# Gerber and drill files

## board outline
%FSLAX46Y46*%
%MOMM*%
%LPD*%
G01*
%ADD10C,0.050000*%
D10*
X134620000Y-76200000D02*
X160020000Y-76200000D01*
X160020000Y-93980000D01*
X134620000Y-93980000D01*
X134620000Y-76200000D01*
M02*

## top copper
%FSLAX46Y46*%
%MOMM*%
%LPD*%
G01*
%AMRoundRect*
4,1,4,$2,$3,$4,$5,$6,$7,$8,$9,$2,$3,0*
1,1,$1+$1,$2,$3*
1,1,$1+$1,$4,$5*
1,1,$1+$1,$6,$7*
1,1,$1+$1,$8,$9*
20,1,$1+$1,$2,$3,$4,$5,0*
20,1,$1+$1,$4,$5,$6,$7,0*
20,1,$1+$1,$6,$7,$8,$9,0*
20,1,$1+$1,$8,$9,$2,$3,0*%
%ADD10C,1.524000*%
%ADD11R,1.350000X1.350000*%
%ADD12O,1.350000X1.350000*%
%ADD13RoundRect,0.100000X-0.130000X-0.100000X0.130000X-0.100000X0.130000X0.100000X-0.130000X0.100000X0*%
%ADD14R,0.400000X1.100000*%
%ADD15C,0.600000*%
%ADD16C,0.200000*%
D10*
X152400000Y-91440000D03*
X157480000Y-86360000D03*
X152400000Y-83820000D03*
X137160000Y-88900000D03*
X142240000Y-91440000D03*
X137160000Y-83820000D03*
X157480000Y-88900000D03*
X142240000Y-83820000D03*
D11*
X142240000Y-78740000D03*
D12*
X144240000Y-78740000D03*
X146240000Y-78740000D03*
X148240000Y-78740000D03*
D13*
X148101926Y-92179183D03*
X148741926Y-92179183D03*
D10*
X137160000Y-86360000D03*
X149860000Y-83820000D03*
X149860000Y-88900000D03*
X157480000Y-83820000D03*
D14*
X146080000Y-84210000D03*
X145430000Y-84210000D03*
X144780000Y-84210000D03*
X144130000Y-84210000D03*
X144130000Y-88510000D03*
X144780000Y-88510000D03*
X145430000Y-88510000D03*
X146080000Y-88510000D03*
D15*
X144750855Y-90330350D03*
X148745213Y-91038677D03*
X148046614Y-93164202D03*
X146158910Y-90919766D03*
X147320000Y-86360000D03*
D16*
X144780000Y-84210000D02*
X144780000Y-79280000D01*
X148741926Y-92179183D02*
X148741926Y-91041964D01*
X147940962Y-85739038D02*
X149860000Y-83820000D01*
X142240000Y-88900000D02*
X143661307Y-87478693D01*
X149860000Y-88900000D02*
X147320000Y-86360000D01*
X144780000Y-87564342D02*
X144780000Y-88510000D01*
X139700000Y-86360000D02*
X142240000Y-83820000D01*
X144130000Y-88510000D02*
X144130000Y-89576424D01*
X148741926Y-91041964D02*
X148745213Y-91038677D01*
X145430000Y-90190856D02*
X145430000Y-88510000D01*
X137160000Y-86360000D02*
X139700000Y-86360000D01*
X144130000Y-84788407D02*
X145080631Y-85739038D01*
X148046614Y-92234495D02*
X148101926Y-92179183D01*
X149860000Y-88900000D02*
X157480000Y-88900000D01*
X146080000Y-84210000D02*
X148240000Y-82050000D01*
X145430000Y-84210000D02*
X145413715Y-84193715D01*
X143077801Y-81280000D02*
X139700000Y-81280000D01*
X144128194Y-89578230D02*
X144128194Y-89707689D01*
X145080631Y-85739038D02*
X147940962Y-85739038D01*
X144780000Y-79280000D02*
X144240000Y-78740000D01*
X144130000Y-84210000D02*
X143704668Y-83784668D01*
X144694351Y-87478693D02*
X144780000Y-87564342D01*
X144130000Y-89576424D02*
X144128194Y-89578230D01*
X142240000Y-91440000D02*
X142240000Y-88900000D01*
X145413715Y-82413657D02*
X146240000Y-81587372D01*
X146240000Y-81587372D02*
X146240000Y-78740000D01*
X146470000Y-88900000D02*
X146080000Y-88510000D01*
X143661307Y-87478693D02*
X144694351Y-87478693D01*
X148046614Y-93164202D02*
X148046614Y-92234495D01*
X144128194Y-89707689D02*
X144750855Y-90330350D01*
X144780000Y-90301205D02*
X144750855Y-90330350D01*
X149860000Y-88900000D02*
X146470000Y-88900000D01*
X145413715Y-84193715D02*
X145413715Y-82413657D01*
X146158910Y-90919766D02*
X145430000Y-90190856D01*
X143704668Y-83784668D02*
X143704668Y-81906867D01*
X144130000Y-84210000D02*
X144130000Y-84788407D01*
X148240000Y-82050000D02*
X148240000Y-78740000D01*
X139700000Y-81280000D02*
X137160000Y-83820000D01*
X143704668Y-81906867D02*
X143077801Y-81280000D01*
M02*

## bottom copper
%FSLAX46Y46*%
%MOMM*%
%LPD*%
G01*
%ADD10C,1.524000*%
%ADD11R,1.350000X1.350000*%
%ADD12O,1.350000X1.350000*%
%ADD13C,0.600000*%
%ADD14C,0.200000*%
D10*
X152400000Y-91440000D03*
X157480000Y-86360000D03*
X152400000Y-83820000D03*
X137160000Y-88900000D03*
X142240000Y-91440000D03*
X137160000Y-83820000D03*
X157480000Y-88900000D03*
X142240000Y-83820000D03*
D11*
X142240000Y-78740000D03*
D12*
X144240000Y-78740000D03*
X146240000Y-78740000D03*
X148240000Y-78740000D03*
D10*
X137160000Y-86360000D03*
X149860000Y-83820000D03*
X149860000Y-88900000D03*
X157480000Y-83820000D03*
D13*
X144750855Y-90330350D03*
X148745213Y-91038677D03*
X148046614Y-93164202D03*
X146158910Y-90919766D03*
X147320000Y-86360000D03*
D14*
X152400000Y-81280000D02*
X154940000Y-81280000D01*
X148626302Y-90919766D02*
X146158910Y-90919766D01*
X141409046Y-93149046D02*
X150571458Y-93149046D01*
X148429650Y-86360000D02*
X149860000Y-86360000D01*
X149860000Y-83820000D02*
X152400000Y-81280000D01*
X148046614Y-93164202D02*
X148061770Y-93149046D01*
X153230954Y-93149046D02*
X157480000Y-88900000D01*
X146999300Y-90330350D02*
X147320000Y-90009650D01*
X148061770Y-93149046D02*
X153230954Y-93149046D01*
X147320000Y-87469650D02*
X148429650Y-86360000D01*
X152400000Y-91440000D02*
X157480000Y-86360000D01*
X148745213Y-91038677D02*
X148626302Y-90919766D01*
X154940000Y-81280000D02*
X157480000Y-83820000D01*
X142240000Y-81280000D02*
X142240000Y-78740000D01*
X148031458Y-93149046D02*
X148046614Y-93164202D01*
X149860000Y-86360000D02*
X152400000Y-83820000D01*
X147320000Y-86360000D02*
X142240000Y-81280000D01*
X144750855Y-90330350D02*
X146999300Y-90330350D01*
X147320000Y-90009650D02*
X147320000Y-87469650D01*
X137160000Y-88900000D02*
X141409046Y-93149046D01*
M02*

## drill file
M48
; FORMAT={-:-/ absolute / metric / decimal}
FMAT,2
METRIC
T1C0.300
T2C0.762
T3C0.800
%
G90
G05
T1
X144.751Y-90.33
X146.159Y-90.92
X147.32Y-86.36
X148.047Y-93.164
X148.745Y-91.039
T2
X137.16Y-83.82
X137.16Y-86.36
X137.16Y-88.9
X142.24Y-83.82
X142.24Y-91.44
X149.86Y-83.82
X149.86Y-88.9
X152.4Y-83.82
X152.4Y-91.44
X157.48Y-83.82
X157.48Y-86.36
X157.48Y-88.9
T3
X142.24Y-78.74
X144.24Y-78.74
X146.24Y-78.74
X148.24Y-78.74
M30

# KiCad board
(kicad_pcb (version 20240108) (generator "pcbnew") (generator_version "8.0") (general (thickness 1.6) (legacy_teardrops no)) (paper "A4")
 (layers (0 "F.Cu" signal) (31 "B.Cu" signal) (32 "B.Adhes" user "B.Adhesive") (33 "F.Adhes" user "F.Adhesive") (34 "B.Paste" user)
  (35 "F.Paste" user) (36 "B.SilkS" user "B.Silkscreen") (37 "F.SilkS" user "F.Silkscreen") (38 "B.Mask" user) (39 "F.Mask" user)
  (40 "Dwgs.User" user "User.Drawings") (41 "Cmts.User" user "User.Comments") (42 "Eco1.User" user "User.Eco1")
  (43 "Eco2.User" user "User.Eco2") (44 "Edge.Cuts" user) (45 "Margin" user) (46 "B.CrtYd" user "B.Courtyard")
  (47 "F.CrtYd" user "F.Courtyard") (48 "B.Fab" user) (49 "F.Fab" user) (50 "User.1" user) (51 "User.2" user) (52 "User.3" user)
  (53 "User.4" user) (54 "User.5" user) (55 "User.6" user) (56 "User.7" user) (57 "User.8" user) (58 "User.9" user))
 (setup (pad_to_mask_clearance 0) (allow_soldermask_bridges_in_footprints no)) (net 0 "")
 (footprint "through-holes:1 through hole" (layer "F.Cu") (at 152.4 91.44)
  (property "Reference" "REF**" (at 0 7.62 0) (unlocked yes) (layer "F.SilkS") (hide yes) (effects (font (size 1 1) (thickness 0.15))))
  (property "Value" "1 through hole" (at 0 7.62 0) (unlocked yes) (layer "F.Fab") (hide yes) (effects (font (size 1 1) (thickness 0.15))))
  (pad "1" thru_hole circle (at 0 0) (size 1.524 1.524) (drill 0.762) (layers "*.Cu" "*.Mask") (remove_unused_layers no)))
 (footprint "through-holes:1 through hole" (layer "F.Cu") (at 157.48 86.36)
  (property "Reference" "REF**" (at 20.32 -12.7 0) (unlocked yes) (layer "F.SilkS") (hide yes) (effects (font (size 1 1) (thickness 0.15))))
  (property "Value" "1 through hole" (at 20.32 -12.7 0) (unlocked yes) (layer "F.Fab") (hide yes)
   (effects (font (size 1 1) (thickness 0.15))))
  (pad "1" thru_hole circle (at 0 0) (size 1.524 1.524) (drill 0.762) (layers "*.Cu" "*.Mask") (remove_unused_layers no)))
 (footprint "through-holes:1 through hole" (layer "F.Cu") (at 152.4 83.82)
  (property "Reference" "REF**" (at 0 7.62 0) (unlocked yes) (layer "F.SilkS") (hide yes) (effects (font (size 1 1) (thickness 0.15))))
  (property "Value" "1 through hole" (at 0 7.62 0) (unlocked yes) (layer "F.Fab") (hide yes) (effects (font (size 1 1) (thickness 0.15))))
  (pad "1" thru_hole circle (at 0 0) (size 1.524 1.524) (drill 0.762) (layers "*.Cu" "*.Mask") (remove_unused_layers no)))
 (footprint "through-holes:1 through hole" (layer "F.Cu") (at 137.16 88.9)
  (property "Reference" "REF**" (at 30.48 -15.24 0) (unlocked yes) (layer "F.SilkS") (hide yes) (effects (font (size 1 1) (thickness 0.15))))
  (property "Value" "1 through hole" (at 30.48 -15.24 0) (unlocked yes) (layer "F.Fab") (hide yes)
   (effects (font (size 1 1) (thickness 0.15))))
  (pad "1" thru_hole circle (at 0 0) (size 1.524 1.524) (drill 0.762) (layers "*.Cu" "*.Mask") (remove_unused_layers no)))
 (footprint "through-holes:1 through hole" (layer "F.Cu") (at 142.24 91.44)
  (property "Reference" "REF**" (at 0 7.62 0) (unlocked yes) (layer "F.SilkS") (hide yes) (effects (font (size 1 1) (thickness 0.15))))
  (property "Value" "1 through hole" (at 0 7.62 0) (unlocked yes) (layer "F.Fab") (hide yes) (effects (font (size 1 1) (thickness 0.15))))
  (pad "1" thru_hole circle (at 0 0) (size 1.524 1.524) (drill 0.762) (layers "*.Cu" "*.Mask") (remove_unused_layers no)))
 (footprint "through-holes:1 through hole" (layer "F.Cu") (at 137.16 83.82)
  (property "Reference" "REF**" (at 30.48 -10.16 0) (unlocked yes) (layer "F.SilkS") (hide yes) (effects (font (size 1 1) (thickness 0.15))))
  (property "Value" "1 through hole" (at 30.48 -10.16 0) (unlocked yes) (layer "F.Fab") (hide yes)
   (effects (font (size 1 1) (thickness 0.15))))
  (pad "1" thru_hole circle (at 0 0) (size 1.524 1.524) (drill 0.762) (layers "*.Cu" "*.Mask") (remove_unused_layers no)))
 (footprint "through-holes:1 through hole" (layer "F.Cu") (at 157.48 88.9)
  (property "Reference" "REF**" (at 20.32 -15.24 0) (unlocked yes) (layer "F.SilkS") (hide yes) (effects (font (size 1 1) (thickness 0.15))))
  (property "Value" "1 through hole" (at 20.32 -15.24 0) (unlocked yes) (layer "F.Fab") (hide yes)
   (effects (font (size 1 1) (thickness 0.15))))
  (pad "1" thru_hole circle (at 0 0) (size 1.524 1.524) (drill 0.762) (layers "*.Cu" "*.Mask") (remove_unused_layers no)))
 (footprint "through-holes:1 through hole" (layer "F.Cu") (at 142.24 83.82)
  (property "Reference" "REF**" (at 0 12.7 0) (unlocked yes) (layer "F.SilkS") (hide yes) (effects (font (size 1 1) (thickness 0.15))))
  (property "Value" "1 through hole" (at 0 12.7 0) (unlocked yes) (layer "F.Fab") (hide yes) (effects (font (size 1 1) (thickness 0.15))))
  (pad "1" thru_hole circle (at 0 0) (size 1.524 1.524) (drill 0.762) (layers "*.Cu" "*.Mask") (remove_unused_layers no)))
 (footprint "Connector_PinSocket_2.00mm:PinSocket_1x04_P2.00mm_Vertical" (layer "F.Cu") (at 142.24 78.74 90)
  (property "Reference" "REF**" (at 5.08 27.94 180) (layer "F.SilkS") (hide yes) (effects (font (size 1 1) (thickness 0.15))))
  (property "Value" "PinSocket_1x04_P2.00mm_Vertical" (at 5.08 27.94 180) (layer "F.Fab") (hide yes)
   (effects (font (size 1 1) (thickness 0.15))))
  (pad "1" thru_hole rect (at 0 0 90) (size 1.35 1.35) (drill 0.8) (layers "*.Cu" "*.Mask") (remove_unused_layers no))
  (pad "2" thru_hole oval (at 0 2 90) (size 1.35 1.35) (drill 0.8) (layers "*.Cu" "*.Mask") (remove_unused_layers no))
  (pad "3" thru_hole oval (at 0 4 90) (size 1.35 1.35) (drill 0.8) (layers "*.Cu" "*.Mask") (remove_unused_layers no))
  (pad "4" thru_hole oval (at 0 6 90) (size 1.35 1.35) (drill 0.8) (layers "*.Cu" "*.Mask") (remove_unused_layers no)))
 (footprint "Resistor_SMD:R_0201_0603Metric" (layer "F.Cu") (at 148.421926 92.179183)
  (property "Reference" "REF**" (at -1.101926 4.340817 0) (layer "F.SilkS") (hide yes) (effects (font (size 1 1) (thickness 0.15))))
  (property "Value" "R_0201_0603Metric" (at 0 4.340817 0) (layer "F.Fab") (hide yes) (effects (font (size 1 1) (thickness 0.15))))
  (pad "" smd roundrect (at -0.345 0) (size 0.318 0.36) (layers "F.Paste") (roundrect_rratio 0.25))
  (pad "" smd roundrect (at 0.345 0) (size 0.318 0.36) (layers "F.Paste") (roundrect_rratio 0.25))
  (pad "1" smd roundrect (at -0.32 0) (size 0.46 0.4) (layers "F.Cu" "F.Mask") (roundrect_rratio 0.25))
  (pad "2" smd roundrect (at 0.32 0) (size 0.46 0.4) (layers "F.Cu" "F.Mask") (roundrect_rratio 0.25)))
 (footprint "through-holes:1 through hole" (layer "F.Cu") (at 137.16 86.36)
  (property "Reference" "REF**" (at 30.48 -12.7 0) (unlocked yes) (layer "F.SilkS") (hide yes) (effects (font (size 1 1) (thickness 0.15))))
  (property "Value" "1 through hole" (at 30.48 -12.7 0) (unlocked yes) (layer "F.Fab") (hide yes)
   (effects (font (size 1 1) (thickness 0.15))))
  (pad "1" thru_hole circle (at 0 0) (size 1.524 1.524) (drill 0.762) (layers "*.Cu" "*.Mask") (remove_unused_layers no)))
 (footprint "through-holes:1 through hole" (layer "F.Cu") (at 149.86 83.82)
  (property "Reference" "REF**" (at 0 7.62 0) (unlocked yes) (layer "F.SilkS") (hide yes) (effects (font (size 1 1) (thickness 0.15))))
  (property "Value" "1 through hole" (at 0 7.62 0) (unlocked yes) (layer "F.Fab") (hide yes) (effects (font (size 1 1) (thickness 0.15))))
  (pad "1" thru_hole circle (at 0 0) (size 1.524 1.524) (drill 0.762) (layers "*.Cu" "*.Mask") (remove_unused_layers no)))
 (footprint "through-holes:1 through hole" (layer "F.Cu") (at 149.86 88.9)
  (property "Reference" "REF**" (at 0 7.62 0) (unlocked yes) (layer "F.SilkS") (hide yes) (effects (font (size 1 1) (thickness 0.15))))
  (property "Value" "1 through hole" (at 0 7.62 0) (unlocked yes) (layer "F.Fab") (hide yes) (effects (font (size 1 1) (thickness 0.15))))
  (pad "1" thru_hole circle (at 0 0) (size 1.524 1.524) (drill 0.762) (layers "*.Cu" "*.Mask") (remove_unused_layers no)))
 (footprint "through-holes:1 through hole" (layer "F.Cu") (at 157.48 83.82)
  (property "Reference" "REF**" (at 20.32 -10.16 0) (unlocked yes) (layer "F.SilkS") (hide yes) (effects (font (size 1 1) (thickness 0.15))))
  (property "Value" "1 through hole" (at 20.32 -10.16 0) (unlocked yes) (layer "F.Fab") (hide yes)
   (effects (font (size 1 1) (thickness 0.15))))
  (pad "1" thru_hole circle (at 0 0) (size 1.524 1.524) (drill 0.762) (layers "*.Cu" "*.Mask") (remove_unused_layers no)))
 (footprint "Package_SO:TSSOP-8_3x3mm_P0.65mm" (layer "F.Cu") (at 145.105 86.36 -90)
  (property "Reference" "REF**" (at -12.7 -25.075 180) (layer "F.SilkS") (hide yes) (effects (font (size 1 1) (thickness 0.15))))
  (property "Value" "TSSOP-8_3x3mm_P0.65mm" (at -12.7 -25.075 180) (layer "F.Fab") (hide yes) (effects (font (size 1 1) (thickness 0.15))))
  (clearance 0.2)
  (pad "1" smd rect (at -2.15 -0.975 270) (size 1.1 0.4) (layers "F.Cu" "F.Paste" "F.Mask"))
  (pad "2" smd rect (at -2.15 -0.325 270) (size 1.1 0.4) (layers "F.Cu" "F.Paste" "F.Mask"))
  (pad "3" smd rect (at -2.15 0.325 270) (size 1.1 0.4) (layers "F.Cu" "F.Paste" "F.Mask"))
  (pad "4" smd rect (at -2.15 0.975 270) (size 1.1 0.4) (layers "F.Cu" "F.Paste" "F.Mask"))
  (pad "5" smd rect (at 2.15 0.975 270) (size 1.1 0.4) (layers "F.Cu" "F.Paste" "F.Mask"))
  (pad "6" smd rect (at 2.15 0.325 270) (size 1.1 0.4) (layers "F.Cu" "F.Paste" "F.Mask"))
  (pad "7" smd rect (at 2.15 -0.325 270) (size 1.1 0.4) (layers "F.Cu" "F.Paste" "F.Mask"))
  (pad "8" smd rect (at 2.15 -0.975 270) (size 1.1 0.4) (layers "F.Cu" "F.Paste" "F.Mask")))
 (gr_rect (start 134.62 76.2) (end 160.02 93.98) (stroke (width 0.05) (type default)) (fill none) (layer "Edge.Cuts"))
 (segment (start 144.78 84.21) (end 144.78 79.28) (width 0.2) (layer "F.Cu") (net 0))
 (segment (start 148.741926 92.179183) (end 148.741926 91.041964) (width 0.2) (layer "F.Cu") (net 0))
 (segment (start 147.940962 85.739038) (end 149.86 83.82) (width 0.2) (layer "F.Cu") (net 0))
 (segment (start 142.24 88.9) (end 143.661307 87.478693) (width 0.2) (layer "F.Cu") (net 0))
 (segment (start 149.86 88.9) (end 147.32 86.36) (width 0.2) (layer "F.Cu") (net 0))
 (segment (start 144.78 87.564342) (end 144.78 88.51) (width 0.2) (layer "F.Cu") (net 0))
 (segment (start 139.7 86.36) (end 142.24 83.82) (width 0.2) (layer "F.Cu") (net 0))
 (segment (start 144.13 88.51) (end 144.13 89.576424) (width 0.2) (layer "F.Cu") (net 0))
 (segment (start 148.741926 91.041964) (end 148.745213 91.038677) (width 0.2) (layer "F.Cu") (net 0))
 (segment (start 145.43 90.190856) (end 145.43 88.51) (width 0.2) (layer "F.Cu") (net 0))
 (segment (start 137.16 86.36) (end 139.7 86.36) (width 0.2) (layer "F.Cu") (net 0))
 (segment (start 144.13 84.788407) (end 145.080631 85.739038) (width 0.2) (layer "F.Cu") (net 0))
 (segment (start 148.046614 92.234495) (end 148.101926 92.179183) (width 0.2) (layer "F.Cu") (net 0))
 (segment (start 149.86 88.9) (end 157.48 88.9) (width 0.2) (layer "F.Cu") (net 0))
 (segment (start 146.08 84.21) (end 148.24 82.05) (width 0.2) (layer "F.Cu") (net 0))
 (segment (start 145.43 84.21) (end 145.413715 84.193715) (width 0.2) (layer "F.Cu") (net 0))
 (segment (start 143.077801 81.28) (end 139.7 81.28) (width 0.2) (layer "F.Cu") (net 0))
 (segment (start 144.128194 89.57823) (end 144.128194 89.707689) (width 0.2) (layer "F.Cu") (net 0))
 (segment (start 145.080631 85.739038) (end 147.940962 85.739038) (width 0.2) (layer "F.Cu") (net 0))
 (segment (start 144.78 79.28) (end 144.24 78.74) (width 0.2) (layer "F.Cu") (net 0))
 (segment (start 144.13 84.21) (end 143.704668 83.784668) (width 0.2) (layer "F.Cu") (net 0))
 (segment (start 144.694351 87.478693) (end 144.78 87.564342) (width 0.2) (layer "F.Cu") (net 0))
 (segment (start 144.13 89.576424) (end 144.128194 89.57823) (width 0.2) (layer "F.Cu") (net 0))
 (segment (start 142.24 91.44) (end 142.24 88.9) (width 0.2) (layer "F.Cu") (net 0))
 (segment (start 145.413715 82.413657) (end 146.24 81.587372) (width 0.2) (layer "F.Cu") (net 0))
 (segment (start 146.24 81.587372) (end 146.24 78.74) (width 0.2) (layer "F.Cu") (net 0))
 (segment (start 146.47 88.9) (end 146.08 88.51) (width 0.2) (layer "F.Cu") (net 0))
 (segment (start 143.661307 87.478693) (end 144.694351 87.478693) (width 0.2) (layer "F.Cu") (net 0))
 (segment (start 148.046614 93.164202) (end 148.046614 92.234495) (width 0.2) (layer "F.Cu") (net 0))
 (segment (start 144.128194 89.707689) (end 144.750855 90.33035) (width 0.2) (layer "F.Cu") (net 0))
 (segment (start 144.78 90.301205) (end 144.750855 90.33035) (width 0.2) (layer "F.Cu") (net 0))
 (segment (start 149.86 88.9) (end 146.47 88.9) (width 0.2) (layer "F.Cu") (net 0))
 (segment (start 145.413715 84.193715) (end 145.413715 82.413657) (width 0.2) (layer "F.Cu") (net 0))
 (segment (start 146.15891 90.919766) (end 145.43 90.190856) (width 0.2) (layer "F.Cu") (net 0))
 (segment (start 143.704668 83.784668) (end 143.704668 81.906867) (width 0.2) (layer "F.Cu") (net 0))
 (segment (start 144.13 84.21) (end 144.13 84.788407) (width 0.2) (layer "F.Cu") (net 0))
 (segment (start 148.24 82.05) (end 148.24 78.74) (width 0.2) (layer "F.Cu") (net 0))
 (segment (start 139.7 81.28) (end 137.16 83.82) (width 0.2) (layer "F.Cu") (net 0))
 (segment (start 143.704668 81.906867) (end 143.077801 81.28) (width 0.2) (layer "F.Cu") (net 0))
 (via (at 144.750855 90.33035) (size 0.6) (drill 0.3) (layers "F.Cu" "B.Cu") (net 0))
 (via (at 148.745213 91.038677) (size 0.6) (drill 0.3) (layers "F.Cu" "B.Cu") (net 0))
 (via (at 148.046614 93.164202) (size 0.6) (drill 0.3) (layers "F.Cu" "B.Cu") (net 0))
 (via (at 146.15891 90.919766) (size 0.6) (drill 0.3) (layers "F.Cu" "B.Cu") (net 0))
 (via (at 147.32 86.36) (size 0.6) (drill 0.3) (layers "F.Cu" "B.Cu") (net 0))
 (segment (start 152.4 81.28) (end 154.94 81.28) (width 0.2) (layer "B.Cu") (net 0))
 (segment (start 148.626302 90.919766) (end 146.15891 90.919766) (width 0.2) (layer "B.Cu") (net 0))
 (segment (start 141.409046 93.149046) (end 150.571458 93.149046) (width 0.2) (layer "B.Cu") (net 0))
 (segment (start 148.42965 86.36) (end 149.86 86.36) (width 0.2) (layer "B.Cu") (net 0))
 (segment (start 149.86 83.82) (end 152.4 81.28) (width 0.2) (layer "B.Cu") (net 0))
 (segment (start 148.046614 93.164202) (end 148.06177 93.149046) (width 0.2) (layer "B.Cu") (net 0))
 (segment (start 153.230954 93.149046) (end 157.48 88.9) (width 0.2) (layer "B.Cu") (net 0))
 (segment (start 146.9993 90.33035) (end 147.32 90.00965) (width 0.2) (layer "B.Cu") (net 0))
 (segment (start 148.06177 93.149046) (end 153.230954 93.149046) (width 0.2) (layer "B.Cu") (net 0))
 (segment (start 147.32 87.46965) (end 148.42965 86.36) (width 0.2) (layer "B.Cu") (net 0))
 (segment (start 152.4 91.44) (end 157.48 86.36) (width 0.2) (layer "B.Cu") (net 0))
 (segment (start 148.745213 91.038677) (end 148.626302 90.919766) (width 0.2) (layer "B.Cu") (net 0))
 (segment (start 154.94 81.28) (end 157.48 83.82) (width 0.2) (layer "B.Cu") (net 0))
 (segment (start 142.24 81.28) (end 142.24 78.74) (width 0.2) (layer "B.Cu") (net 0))
 (segment (start 148.031458 93.149046) (end 148.046614 93.164202) (width 0.2) (layer "B.Cu") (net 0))
 (segment (start 149.86 86.36) (end 152.4 83.82) (width 0.2) (layer "B.Cu") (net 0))
 (segment (start 147.32 86.36) (end 142.24 81.28) (width 0.2) (layer "B.Cu") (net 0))
 (segment (start 144.750855 90.33035) (end 146.9993 90.33035) (width 0.2) (layer "B.Cu") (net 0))
 (segment (start 147.32 90.00965) (end 147.32 87.46965) (width 0.2) (layer "B.Cu") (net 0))
 (segment (start 137.16 88.9) (end 141.409046 93.149046) (width 0.2) (layer "B.Cu") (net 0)))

